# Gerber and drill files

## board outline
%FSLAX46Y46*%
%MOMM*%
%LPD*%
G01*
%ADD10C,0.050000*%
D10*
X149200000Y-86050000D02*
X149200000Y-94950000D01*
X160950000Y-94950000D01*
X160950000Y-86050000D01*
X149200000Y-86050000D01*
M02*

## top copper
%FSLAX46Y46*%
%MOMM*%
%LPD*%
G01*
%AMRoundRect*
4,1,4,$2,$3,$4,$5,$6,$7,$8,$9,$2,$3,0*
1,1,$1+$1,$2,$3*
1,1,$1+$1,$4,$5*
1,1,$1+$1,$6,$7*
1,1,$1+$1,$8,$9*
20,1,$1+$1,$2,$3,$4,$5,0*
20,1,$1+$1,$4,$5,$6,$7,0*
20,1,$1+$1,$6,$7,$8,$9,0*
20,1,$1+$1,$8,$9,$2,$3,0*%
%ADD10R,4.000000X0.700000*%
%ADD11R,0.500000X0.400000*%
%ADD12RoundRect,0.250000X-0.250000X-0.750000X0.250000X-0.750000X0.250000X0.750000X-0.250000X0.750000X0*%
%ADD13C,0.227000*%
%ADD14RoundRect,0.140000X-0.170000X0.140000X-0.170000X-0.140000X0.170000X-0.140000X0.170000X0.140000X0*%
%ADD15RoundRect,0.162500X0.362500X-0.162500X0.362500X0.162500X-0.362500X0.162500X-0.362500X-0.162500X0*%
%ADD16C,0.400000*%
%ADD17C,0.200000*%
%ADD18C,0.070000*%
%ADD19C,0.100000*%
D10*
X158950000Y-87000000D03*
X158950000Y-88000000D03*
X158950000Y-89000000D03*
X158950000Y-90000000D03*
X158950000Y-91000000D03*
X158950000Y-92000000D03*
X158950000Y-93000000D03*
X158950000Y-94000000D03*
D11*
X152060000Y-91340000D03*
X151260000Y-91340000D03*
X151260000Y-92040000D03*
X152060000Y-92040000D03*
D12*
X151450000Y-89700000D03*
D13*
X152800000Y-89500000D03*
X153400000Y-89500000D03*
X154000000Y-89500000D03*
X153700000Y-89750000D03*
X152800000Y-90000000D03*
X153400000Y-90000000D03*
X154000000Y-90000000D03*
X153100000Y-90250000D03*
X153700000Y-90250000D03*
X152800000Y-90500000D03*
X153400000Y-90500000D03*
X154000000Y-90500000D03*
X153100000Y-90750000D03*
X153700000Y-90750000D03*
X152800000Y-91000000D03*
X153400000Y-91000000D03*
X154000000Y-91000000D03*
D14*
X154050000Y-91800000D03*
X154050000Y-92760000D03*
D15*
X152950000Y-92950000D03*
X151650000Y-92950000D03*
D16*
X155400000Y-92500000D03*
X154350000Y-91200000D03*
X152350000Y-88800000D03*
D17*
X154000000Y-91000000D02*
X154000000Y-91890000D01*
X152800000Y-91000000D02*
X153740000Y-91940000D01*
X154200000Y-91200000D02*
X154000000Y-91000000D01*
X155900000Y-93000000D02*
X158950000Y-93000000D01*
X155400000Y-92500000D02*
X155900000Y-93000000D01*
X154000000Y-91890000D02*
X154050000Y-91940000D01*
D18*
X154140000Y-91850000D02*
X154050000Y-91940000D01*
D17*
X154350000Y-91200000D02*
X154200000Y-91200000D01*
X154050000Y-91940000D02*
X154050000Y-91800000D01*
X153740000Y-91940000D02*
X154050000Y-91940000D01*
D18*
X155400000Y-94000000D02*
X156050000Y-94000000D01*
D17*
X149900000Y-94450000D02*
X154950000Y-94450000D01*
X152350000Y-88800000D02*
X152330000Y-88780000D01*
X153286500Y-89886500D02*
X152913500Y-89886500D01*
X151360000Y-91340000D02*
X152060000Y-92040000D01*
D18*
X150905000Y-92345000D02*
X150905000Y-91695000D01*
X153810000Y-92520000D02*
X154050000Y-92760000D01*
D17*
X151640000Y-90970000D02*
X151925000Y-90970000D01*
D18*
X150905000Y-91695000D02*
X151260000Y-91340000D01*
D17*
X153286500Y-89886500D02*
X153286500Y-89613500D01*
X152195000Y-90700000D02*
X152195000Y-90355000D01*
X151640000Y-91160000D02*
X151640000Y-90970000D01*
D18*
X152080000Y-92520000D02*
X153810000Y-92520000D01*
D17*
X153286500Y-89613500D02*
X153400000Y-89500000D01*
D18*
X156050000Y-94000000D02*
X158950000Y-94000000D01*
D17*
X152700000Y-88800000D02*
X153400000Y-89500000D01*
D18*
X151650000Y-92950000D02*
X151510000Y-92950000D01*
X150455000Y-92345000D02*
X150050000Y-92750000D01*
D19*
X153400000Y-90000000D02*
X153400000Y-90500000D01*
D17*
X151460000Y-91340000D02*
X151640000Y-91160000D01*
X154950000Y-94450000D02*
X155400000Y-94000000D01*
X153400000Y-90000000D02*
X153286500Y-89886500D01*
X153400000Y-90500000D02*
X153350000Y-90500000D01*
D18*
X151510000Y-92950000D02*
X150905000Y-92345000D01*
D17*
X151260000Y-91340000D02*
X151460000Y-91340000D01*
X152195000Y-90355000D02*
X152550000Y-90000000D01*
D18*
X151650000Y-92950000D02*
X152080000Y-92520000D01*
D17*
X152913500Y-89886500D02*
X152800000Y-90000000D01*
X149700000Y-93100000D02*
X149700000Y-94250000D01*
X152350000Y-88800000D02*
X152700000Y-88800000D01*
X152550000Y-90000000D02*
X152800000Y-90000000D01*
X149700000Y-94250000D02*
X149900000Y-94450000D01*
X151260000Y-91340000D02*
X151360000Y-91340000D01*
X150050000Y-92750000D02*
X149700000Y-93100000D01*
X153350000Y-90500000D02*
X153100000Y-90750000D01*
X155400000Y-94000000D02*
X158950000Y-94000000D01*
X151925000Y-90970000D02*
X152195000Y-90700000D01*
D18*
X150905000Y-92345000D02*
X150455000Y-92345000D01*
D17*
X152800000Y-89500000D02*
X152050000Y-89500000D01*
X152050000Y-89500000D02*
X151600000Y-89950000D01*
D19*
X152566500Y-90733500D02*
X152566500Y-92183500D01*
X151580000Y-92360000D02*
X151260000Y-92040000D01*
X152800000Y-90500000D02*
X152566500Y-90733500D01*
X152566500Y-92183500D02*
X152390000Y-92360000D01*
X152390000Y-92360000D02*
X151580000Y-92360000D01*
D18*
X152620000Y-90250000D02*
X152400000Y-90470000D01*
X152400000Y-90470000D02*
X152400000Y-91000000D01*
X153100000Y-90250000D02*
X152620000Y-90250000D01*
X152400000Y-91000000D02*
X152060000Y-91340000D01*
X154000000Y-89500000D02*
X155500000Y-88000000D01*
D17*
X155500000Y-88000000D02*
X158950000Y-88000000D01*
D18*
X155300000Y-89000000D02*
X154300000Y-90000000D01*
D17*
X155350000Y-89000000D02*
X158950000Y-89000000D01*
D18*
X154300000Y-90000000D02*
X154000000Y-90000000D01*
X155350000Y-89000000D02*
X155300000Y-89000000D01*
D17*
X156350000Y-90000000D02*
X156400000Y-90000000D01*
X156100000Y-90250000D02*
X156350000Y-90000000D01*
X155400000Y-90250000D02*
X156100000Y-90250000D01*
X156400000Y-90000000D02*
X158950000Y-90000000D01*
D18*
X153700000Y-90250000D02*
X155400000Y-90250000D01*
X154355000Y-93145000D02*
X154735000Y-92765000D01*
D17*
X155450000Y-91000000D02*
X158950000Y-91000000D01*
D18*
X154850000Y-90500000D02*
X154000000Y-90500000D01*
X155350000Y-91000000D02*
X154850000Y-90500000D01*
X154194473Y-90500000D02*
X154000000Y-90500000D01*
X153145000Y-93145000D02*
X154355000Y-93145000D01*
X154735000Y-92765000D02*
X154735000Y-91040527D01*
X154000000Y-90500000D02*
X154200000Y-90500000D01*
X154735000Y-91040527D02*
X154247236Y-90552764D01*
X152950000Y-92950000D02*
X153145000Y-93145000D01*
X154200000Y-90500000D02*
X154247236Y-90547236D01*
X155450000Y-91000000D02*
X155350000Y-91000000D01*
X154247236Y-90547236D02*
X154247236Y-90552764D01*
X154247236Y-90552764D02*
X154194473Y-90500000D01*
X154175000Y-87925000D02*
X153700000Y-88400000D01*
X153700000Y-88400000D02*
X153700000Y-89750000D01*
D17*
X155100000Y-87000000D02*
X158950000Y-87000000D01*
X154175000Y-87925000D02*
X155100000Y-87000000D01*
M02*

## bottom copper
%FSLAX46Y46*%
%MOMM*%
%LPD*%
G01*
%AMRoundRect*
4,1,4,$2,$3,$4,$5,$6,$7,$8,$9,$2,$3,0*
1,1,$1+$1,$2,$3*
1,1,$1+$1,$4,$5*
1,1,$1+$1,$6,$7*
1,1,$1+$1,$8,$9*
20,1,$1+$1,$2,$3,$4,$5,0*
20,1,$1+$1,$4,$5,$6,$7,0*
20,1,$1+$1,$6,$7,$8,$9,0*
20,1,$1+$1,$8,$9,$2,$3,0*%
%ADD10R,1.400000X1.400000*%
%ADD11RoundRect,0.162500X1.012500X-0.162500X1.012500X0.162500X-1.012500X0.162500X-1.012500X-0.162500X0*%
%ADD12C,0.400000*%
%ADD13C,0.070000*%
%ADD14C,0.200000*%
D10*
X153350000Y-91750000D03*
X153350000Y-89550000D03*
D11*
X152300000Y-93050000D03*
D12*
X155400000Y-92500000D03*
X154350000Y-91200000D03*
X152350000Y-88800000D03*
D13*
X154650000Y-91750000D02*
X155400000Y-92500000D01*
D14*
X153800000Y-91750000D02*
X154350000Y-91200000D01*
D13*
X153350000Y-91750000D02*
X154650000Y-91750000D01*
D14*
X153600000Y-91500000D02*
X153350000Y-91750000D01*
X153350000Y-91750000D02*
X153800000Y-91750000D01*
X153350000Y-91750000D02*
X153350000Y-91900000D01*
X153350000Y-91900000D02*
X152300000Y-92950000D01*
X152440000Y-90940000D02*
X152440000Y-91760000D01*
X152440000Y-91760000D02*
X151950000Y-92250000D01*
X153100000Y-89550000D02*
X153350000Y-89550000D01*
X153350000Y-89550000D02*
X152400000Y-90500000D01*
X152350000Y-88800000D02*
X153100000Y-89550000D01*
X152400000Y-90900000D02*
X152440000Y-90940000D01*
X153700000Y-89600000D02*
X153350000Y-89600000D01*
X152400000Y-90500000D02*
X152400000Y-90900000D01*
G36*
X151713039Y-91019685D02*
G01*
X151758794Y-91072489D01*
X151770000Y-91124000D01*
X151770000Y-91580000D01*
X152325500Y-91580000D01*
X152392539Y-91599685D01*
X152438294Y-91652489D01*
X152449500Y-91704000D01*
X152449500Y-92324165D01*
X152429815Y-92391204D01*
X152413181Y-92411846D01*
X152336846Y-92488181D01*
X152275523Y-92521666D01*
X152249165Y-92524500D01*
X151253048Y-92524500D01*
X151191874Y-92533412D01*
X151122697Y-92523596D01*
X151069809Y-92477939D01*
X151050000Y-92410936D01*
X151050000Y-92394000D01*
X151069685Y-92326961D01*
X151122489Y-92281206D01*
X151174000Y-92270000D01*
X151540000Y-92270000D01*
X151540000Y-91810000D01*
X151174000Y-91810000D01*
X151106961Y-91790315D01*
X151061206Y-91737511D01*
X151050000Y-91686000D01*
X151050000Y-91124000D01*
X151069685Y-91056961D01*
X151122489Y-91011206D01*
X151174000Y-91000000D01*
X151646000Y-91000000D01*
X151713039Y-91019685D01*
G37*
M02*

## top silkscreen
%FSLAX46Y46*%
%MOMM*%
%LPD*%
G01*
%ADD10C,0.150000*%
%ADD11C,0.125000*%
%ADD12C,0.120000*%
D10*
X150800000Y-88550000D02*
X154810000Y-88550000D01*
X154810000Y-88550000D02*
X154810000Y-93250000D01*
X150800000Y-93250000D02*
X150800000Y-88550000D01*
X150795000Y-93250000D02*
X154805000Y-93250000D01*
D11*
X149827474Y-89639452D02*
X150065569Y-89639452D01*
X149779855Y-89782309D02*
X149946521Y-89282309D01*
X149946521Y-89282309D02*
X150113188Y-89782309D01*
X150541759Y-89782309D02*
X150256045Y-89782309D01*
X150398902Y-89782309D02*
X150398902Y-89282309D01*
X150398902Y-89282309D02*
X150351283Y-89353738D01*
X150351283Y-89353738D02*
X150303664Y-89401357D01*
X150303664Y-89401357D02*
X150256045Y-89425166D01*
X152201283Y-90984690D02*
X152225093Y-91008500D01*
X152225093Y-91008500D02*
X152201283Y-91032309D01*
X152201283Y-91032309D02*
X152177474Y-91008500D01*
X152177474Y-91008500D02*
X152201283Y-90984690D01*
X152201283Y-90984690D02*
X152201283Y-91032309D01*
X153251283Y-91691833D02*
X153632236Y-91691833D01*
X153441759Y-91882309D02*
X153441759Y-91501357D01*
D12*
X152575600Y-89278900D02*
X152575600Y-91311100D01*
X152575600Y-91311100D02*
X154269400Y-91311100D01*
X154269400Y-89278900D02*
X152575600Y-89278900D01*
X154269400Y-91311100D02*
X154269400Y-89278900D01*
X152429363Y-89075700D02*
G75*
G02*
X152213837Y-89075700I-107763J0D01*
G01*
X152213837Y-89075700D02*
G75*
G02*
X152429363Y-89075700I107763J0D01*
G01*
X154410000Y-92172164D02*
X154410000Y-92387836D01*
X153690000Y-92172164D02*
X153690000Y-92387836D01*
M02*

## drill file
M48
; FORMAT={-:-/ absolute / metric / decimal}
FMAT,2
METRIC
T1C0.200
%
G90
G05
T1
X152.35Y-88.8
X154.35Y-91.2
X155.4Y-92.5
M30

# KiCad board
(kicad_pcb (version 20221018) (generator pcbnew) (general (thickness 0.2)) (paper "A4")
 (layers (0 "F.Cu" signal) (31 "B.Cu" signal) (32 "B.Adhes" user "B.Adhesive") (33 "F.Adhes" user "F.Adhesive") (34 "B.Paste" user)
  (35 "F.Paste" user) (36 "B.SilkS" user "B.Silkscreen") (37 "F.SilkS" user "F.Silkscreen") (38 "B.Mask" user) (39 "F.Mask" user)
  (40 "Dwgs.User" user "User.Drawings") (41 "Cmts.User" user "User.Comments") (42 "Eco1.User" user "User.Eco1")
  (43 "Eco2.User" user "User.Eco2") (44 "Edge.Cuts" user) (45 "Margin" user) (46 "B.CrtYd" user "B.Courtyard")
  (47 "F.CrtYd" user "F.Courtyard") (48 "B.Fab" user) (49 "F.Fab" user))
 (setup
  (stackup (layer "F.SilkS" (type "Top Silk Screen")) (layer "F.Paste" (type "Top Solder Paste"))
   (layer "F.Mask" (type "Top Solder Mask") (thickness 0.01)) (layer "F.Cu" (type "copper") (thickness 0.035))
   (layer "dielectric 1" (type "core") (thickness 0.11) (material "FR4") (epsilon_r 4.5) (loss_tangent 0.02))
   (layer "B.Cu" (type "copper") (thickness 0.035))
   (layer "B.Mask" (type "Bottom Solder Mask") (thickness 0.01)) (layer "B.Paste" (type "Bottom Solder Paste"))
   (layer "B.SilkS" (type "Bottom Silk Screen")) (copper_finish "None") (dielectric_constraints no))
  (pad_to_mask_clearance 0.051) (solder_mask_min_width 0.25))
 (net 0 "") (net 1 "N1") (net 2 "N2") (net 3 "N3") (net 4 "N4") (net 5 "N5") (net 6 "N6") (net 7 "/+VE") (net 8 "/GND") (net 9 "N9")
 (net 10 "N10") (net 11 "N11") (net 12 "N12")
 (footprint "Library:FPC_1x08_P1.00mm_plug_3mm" (layer "F.Cu") (at 156.95 90.5)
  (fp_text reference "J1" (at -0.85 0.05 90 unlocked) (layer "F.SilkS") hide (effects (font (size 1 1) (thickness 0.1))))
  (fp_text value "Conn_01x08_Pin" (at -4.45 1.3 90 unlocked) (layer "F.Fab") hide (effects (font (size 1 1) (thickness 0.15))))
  (pad "1" connect rect (at 2 -3.5) (size 4 0.7) (layers "F.Cu" "F.Mask") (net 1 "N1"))
  (pad "2" connect rect (at 2 -2.5) (size 4 0.7) (layers "F.Cu" "F.Mask") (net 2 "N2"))
  (pad "3" connect rect (at 2 -1.5) (size 4 0.7) (layers "F.Cu" "F.Mask") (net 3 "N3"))
  (pad "4" connect rect (at 2 -0.5) (size 4 0.7) (layers "F.Cu" "F.Mask") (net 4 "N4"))
  (pad "5" connect rect (at 2 0.5) (size 4 0.7) (layers "F.Cu" "F.Mask") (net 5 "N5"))
  (pad "6" connect rect (at 2 1.5) (size 4 0.7) (layers "F.Cu" "F.Mask") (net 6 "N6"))
  (pad "7" connect rect (at 2 2.5) (size 4 0.7) (layers "F.Cu" "F.Mask") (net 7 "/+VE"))
  (pad "8" connect rect (at 2 3.5) (size 4 0.7) (layers "F.Cu" "F.Mask") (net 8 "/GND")))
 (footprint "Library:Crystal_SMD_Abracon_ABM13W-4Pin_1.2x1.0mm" (layer "F.Cu") (at 151.66 91.69 180)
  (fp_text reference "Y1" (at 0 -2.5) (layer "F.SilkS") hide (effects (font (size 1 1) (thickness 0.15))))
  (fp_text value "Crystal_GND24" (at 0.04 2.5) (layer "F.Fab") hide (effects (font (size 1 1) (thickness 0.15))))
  (pad "1" smd rect (at -0.4 0.35 180) (size 0.5 0.4) (layers "F.Cu" "F.Paste" "F.Mask") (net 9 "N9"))
  (pad "2" smd rect (at 0.4 0.35 180) (size 0.5 0.4) (layers "F.Cu" "F.Paste" "F.Mask") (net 8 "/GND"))
  (pad "3" smd rect (at 0.4 -0.35 180) (size 0.5 0.4) (layers "F.Cu" "F.Paste" "F.Mask") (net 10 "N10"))
  (pad "4" smd rect (at -0.4 -0.35 180) (size 0.5 0.4) (layers "F.Cu" "F.Paste" "F.Mask") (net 8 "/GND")))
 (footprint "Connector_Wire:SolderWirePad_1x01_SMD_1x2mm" (layer "F.Cu") (at 151.45 89.7)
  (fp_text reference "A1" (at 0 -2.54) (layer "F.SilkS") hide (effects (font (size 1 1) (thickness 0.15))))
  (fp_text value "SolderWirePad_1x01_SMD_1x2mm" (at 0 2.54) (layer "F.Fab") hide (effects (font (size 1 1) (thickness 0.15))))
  (pad "1" smd roundrect (at 0 0) (size 1 2) (layers "F.Cu" "F.Paste" "F.Mask") (roundrect_rratio 0.25) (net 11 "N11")))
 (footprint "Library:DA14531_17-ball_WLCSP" (layer "F.Cu") (at 153.422 90.295)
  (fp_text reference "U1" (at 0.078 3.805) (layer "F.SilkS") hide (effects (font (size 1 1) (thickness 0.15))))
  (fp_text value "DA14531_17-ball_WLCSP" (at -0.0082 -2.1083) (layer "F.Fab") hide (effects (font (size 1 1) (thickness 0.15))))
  (fp_line (start -0.8464 -1.0161) (end -0.8464 1.0161) (stroke (width 0.12) (type solid)) (layer "F.SilkS"))
  (fp_line (start -0.8464 1.0161) (end 0.8474 1.0161) (stroke (width 0.12) (type solid)) (layer "F.SilkS"))
  (fp_line (start 0.8474 -1.0161) (end -0.8464 -1.0161) (stroke (width 0.12) (type solid)) (layer "F.SilkS"))
  (fp_line (start 0.8474 1.0161) (end 0.8474 -1.0161) (stroke (width 0.12) (type solid)) (layer "F.SilkS"))
  (fp_circle (center -1.1004 -1.2193) (end -1.0242 -1.1431) (stroke (width 0.12) (type solid)) (fill none) (layer "F.SilkS"))
  (pad "A1" smd circle (at -0.622 -0.795) (size 0.227 0.227) (layers "F.Cu" "F.Paste" "F.Mask") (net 11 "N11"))
  (pad "A3" smd circle (at -0.022 -0.795) (size 0.227 0.227) (layers "F.Cu" "F.Paste" "F.Mask") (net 8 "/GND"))
  (pad "A5" smd circle (at 0.578 -0.795) (size 0.227 0.227) (layers "F.Cu" "F.Paste" "F.Mask") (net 2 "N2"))
  (pad "B4" smd circle (at 0.278 -0.545) (size 0.227 0.227) (layers "F.Cu" "F.Paste" "F.Mask") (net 1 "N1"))
  (pad "C1" smd circle (at -0.622 -0.295) (size 0.227 0.227) (layers "F.Cu" "F.Paste" "F.Mask") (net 8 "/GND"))
  (pad "C3" smd circle (at -0.022 -0.295) (size 0.227 0.227) (layers "F.Cu" "F.Paste" "F.Mask") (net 8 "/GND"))
  (pad "C5" smd circle (at 0.578 -0.295) (size 0.227 0.227) (layers "F.Cu" "F.Paste" "F.Mask") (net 3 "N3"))
  (pad "D2" smd circle (at -0.322 -0.045) (size 0.227 0.227) (layers "F.Cu" "F.Paste" "F.Mask") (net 9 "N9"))
  (pad "D4" smd circle (at 0.278 -0.045) (size 0.227 0.227) (layers "F.Cu" "F.Paste" "F.Mask") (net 4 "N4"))
  (pad "E1" smd circle (at -0.622 0.205) (size 0.227 0.227) (layers "F.Cu" "F.Paste" "F.Mask") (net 10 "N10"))
  (pad "E3" smd circle (at -0.022 0.205) (size 0.227 0.227) (layers "F.Cu" "F.Paste" "F.Mask") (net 8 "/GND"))
  (pad "E5" smd circle (at 0.578 0.205) (size 0.227 0.227) (layers "F.Cu" "F.Paste" "F.Mask") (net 5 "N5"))
  (pad "F2" smd circle (at -0.322 0.455) (size 0.227 0.227) (layers "F.Cu" "F.Paste" "F.Mask") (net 8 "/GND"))
  (pad "F4" smd circle (at 0.278 0.455) (size 0.227 0.227) (layers "F.Cu" "F.Paste" "F.Mask") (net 6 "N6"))
  (pad "G1" smd circle (at -0.622 0.705) (size 0.227 0.227) (layers "F.Cu" "F.Paste" "F.Mask") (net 7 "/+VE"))
  (pad "G3" smd circle (at -0.022 0.705) (size 0.227 0.227) (layers "F.Cu" "F.Paste" "F.Mask") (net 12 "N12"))
  (pad "G5" smd circle (at 0.578 0.705) (size 0.227 0.227) (layers "F.Cu" "F.Paste" "F.Mask") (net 7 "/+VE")))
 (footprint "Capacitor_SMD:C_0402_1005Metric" (layer "F.Cu") (at 154.05 92.28 -90)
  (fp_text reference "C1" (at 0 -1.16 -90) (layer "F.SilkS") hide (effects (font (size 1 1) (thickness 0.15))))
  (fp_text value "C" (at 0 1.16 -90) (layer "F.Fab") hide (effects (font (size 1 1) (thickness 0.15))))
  (fp_line (start -0.107836 -0.36) (end 0.107836 -0.36) (stroke (width 0.12) (type solid)) (layer "F.SilkS"))
  (fp_line (start -0.107836 0.36) (end 0.107836 0.36) (stroke (width 0.12) (type solid)) (layer "F.SilkS"))
  (pad "1" smd roundrect (at -0.48 0 270) (size 0.56 0.62) (layers "F.Cu" "F.Paste" "F.Mask") (roundrect_rratio 0.25) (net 7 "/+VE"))
  (pad "2" smd roundrect (at 0.48 0 270) (size 0.56 0.62) (layers "F.Cu" "F.Paste" "F.Mask") (roundrect_rratio 0.25) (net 8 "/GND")))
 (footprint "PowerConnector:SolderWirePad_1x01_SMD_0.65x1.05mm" (layer "F.Cu") (at 152.95 92.95 90)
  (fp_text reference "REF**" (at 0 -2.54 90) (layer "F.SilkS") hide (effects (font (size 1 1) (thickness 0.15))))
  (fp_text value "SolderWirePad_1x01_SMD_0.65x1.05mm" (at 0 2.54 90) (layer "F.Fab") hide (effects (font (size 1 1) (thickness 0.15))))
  (pad "1" smd roundrect (at 0 0 90) (size 0.65 1.05) (layers "F.Cu" "F.Paste" "F.Mask") (roundrect_rratio 0.25) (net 5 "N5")))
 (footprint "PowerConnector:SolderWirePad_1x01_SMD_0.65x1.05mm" (layer "F.Cu") (at 151.65 92.95 90)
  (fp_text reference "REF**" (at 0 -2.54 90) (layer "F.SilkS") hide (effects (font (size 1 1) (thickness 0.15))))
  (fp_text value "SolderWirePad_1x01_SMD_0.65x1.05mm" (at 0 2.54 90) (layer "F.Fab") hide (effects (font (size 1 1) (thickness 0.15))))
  (pad "1" smd roundrect (at 0 0 90) (size 0.65 1.05) (layers "F.Cu" "F.Paste" "F.Mask") (roundrect_rratio 0.25) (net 8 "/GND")))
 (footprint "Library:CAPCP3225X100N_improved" (layer "B.Cu") (at 153.35 90.65 90)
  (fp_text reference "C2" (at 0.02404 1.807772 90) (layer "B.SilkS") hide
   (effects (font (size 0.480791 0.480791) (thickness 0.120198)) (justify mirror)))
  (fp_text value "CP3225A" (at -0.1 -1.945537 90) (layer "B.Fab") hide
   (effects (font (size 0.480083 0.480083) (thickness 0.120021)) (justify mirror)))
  (pad "1" smd rect (at -1.1 0 270) (size 1.4 1.4) (layers "B.Cu" "B.Paste" "B.Mask") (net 7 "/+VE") (solder_mask_margin 0.102))
  (pad "2" smd rect (at 1.1 0 270) (size 1.4 1.4) (layers "B.Cu" "B.Paste" "B.Mask") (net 8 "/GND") (solder_mask_margin 0.102)))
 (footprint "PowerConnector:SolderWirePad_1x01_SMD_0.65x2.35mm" (layer "B.Cu") (at 152.3 93.05 90)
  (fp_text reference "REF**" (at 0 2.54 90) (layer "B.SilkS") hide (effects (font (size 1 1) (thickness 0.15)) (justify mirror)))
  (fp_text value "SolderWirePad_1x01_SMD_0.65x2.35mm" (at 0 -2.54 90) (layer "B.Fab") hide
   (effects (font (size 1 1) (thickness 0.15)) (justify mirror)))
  (pad "1" smd roundrect (at 0 0 90) (size 0.65 2.35) (layers "B.Cu" "B.Paste" "B.Mask") (roundrect_rratio 0.25) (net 7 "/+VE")))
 (gr_line (start 150.8 88.55) (end 154.81 88.55) (stroke (width 0.15) (type default)) (layer "F.SilkS"))
 (gr_line (start 154.81 88.55) (end 154.81 93.25) (stroke (width 0.15) (type default)) (layer "F.SilkS"))
 (gr_line (start 150.8 93.25) (end 150.8 88.55) (stroke (width 0.15) (type default)) (layer "F.SilkS"))
 (gr_line (start 150.795 93.25) (end 154.805 93.25) (stroke (width 0.15) (type default)) (layer "F.SilkS"))
 (gr_poly
  (pts (xy 149.2 86.05) (xy 149.2 94.95) (xy 160.95 94.95) (xy 160.95 86.05)) (stroke (width 0.05) (type solid)) (fill none)
  (layer "Edge.Cuts"))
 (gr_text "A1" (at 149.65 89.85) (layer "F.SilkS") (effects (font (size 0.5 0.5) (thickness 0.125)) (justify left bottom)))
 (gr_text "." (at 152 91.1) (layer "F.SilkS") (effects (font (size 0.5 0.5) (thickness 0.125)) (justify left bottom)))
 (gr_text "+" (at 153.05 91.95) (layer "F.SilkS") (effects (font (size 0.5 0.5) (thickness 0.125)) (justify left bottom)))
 (segment (start 154 91) (end 154 91.89) (width 0.2) (layer "F.Cu") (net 7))
 (segment (start 152.8 91) (end 153.74 91.94) (width 0.2) (layer "F.Cu") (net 7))
 (segment (start 154.2 91.2) (end 154 91) (width 0.2) (layer "F.Cu") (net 7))
 (segment (start 155.9 93) (end 158.95 93) (width 0.2) (layer "F.Cu") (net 7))
 (segment (start 155.4 92.5) (end 155.9 93) (width 0.2) (layer "F.Cu") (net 7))
 (segment (start 154 91.89) (end 154.05 91.94) (width 0.2) (layer "F.Cu") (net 7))
 (segment (start 154.14 91.85) (end 154.05 91.94) (width 0.07) (layer "F.Cu") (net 7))
 (segment (start 154.35 91.2) (end 154.2 91.2) (width 0.2) (layer "F.Cu") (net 7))
 (segment (start 154.05 91.94) (end 154.05 91.8) (width 0.2) (layer "F.Cu") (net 7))
 (segment (start 153.74 91.94) (end 154.05 91.94) (width 0.2) (layer "F.Cu") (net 7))
 (via (at 155.4 92.5) (size 0.4) (drill 0.2) (layers "F.Cu" "B.Cu") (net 7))
 (via (at 154.35 91.2) (size 0.4) (drill 0.2) (layers "F.Cu" "B.Cu") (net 7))
 (segment (start 154.65 91.75) (end 155.4 92.5) (width 0.07) (layer "B.Cu") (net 7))
 (segment (start 153.8 91.75) (end 154.35 91.2) (width 0.2) (layer "B.Cu") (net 7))
 (segment (start 153.35 91.75) (end 154.65 91.75) (width 0.07) (layer "B.Cu") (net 7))
 (segment (start 153.6 91.5) (end 153.35 91.75) (width 0.2) (layer "B.Cu") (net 7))
 (segment (start 153.35 91.75) (end 153.8 91.75) (width 0.2) (layer "B.Cu") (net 7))
 (segment (start 153.35 91.75) (end 153.35 91.9) (width 0.2) (layer "B.Cu") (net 7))
 (segment (start 153.35 91.9) (end 152.3 92.95) (width 0.2) (layer "B.Cu") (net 7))
 (segment (start 155.4 94) (end 156.05 94) (width 0.07) (layer "F.Cu") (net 8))
 (segment (start 149.9 94.45) (end 154.95 94.45) (width 0.2) (layer "F.Cu") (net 8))
 (segment (start 152.35 88.8) (end 152.33 88.78) (width 0.2) (layer "F.Cu") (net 8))
 (segment (start 153.2865 89.8865) (end 152.9135 89.8865) (width 0.2) (layer "F.Cu") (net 8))
 (segment (start 151.36 91.34) (end 152.06 92.04) (width 0.2) (layer "F.Cu") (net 8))
 (segment (start 150.905 92.345) (end 150.905 91.695) (width 0.07) (layer "F.Cu") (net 8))
 (segment (start 153.81 92.52) (end 154.05 92.76) (width 0.07) (layer "F.Cu") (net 8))
 (segment (start 151.64 90.97) (end 151.925 90.97) (width 0.2) (layer "F.Cu") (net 8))
 (segment (start 150.905 91.695) (end 151.26 91.34) (width 0.07) (layer "F.Cu") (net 8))
 (segment (start 153.2865 89.8865) (end 153.2865 89.6135) (width 0.2) (layer "F.Cu") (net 8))
 (segment (start 152.195 90.7) (end 152.195 90.355) (width 0.2) (layer "F.Cu") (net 8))
 (segment (start 151.64 91.16) (end 151.64 90.97) (width 0.2) (layer "F.Cu") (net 8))
 (segment (start 152.08 92.52) (end 153.81 92.52) (width 0.07) (layer "F.Cu") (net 8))
 (segment (start 153.2865 89.6135) (end 153.4 89.5) (width 0.2) (layer "F.Cu") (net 8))
 (segment (start 156.05 94) (end 158.95 94) (width 0.07) (layer "F.Cu") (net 8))
 (segment (start 152.7 88.8) (end 153.4 89.5) (width 0.2) (layer "F.Cu") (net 8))
 (segment (start 151.65 92.95) (end 151.51 92.95) (width 0.07) (layer "F.Cu") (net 8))
 (segment (start 150.455 92.345) (end 150.05 92.75) (width 0.07) (layer "F.Cu") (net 8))
 (segment (start 153.4 90) (end 153.4 90.5) (width 0.1) (layer "F.Cu") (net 8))
 (segment (start 151.46 91.34) (end 151.64 91.16) (width 0.2) (layer "F.Cu") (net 8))
 (segment (start 154.95 94.45) (end 155.4 94) (width 0.2) (layer "F.Cu") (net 8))
 (segment (start 153.4 90) (end 153.2865 89.8865) (width 0.2) (layer "F.Cu") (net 8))
 (segment (start 153.4 90.5) (end 153.35 90.5) (width 0.2) (layer "F.Cu") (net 8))
 (segment (start 151.51 92.95) (end 150.905 92.345) (width 0.07) (layer "F.Cu") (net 8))
 (segment (start 151.26 91.34) (end 151.46 91.34) (width 0.2) (layer "F.Cu") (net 8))
 (segment (start 152.195 90.355) (end 152.55 90) (width 0.2) (layer "F.Cu") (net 8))
 (segment (start 151.65 92.95) (end 152.08 92.52) (width 0.07) (layer "F.Cu") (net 8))
 (segment (start 152.9135 89.8865) (end 152.8 90) (width 0.2) (layer "F.Cu") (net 8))
 (segment (start 149.7 93.1) (end 149.7 94.25) (width 0.2) (layer "F.Cu") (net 8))
 (segment (start 152.35 88.8) (end 152.7 88.8) (width 0.2) (layer "F.Cu") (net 8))
 (segment (start 152.55 90) (end 152.8 90) (width 0.2) (layer "F.Cu") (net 8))
 (segment (start 149.7 94.25) (end 149.9 94.45) (width 0.2) (layer "F.Cu") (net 8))
 (segment (start 151.26 91.34) (end 151.36 91.34) (width 0.2) (layer "F.Cu") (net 8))
 (segment (start 150.05 92.75) (end 149.7 93.1) (width 0.2) (layer "F.Cu") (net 8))
 (segment (start 153.35 90.5) (end 153.1 90.75) (width 0.2) (layer "F.Cu") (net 8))
 (segment (start 155.4 94) (end 158.95 94) (width 0.2) (layer "F.Cu") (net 8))
 (segment (start 151.925 90.97) (end 152.195 90.7) (width 0.2) (layer "F.Cu") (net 8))
 (segment (start 150.905 92.345) (end 150.455 92.345) (width 0.07) (layer "F.Cu") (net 8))
 (via (at 152.35 88.8) (size 0.4) (drill 0.2) (layers "F.Cu" "B.Cu") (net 8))
 (segment (start 152.44 90.94) (end 152.44 91.76) (width 0.2) (layer "B.Cu") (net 8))
 (segment (start 152.44 91.76) (end 151.95 92.25) (width 0.2) (layer "B.Cu") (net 8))
 (segment (start 153.1 89.55) (end 153.35 89.55) (width 0.2) (layer "B.Cu") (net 8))
 (segment (start 153.35 89.55) (end 152.4 90.5) (width 0.2) (layer "B.Cu") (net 8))
 (segment (start 152.35 88.8) (end 153.1 89.55) (width 0.2) (layer "B.Cu") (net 8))
 (segment (start 152.4 90.9) (end 152.44 90.94) (width 0.2) (layer "B.Cu") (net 8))
 (segment (start 153.7 89.6) (end 153.35 89.6) (width 0.2) (layer "B.Cu") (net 8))
 (segment (start 152.4 90.5) (end 152.4 90.9) (width 0.2) (layer "B.Cu") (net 8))
 (segment (start 152.8 89.5) (end 152.05 89.5) (width 0.2) (layer "F.Cu") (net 11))
 (segment (start 152.05 89.5) (end 151.6 89.95) (width 0.2) (layer "F.Cu") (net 11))
 (segment (start 152.5665 90.7335) (end 152.5665 92.1835) (width 0.1) (layer "F.Cu") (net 10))
 (segment (start 151.58 92.36) (end 151.26 92.04) (width 0.1) (layer "F.Cu") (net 10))
 (segment (start 152.8 90.5) (end 152.5665 90.7335) (width 0.1) (layer "F.Cu") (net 10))
 (segment (start 152.5665 92.1835) (end 152.39 92.36) (width 0.1) (layer "F.Cu") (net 10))
 (segment (start 152.39 92.36) (end 151.58 92.36) (width 0.1) (layer "F.Cu") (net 10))
 (segment (start 152.62 90.25) (end 152.4 90.47) (width 0.07) (layer "F.Cu") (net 9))
 (segment (start 152.4 90.47) (end 152.4 91) (width 0.07) (layer "F.Cu") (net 9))
 (segment (start 153.1 90.25) (end 152.62 90.25) (width 0.07) (layer "F.Cu") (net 9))
 (segment (start 152.4 91) (end 152.06 91.34) (width 0.07) (layer "F.Cu") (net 9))
 (segment (start 154 89.5) (end 155.5 88) (width 0.07) (layer "F.Cu") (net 2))
 (segment (start 155.5 88) (end 158.95 88) (width 0.2) (layer "F.Cu") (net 2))
 (segment (start 155.3 89) (end 154.3 90) (width 0.07) (layer "F.Cu") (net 3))
 (segment (start 155.35 89) (end 158.95 89) (width 0.2) (layer "F.Cu") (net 3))
 (segment (start 154.3 90) (end 154 90) (width 0.07) (layer "F.Cu") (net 3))
 (segment (start 155.35 89) (end 155.3 89) (width 0.07) (layer "F.Cu") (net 3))
 (segment (start 156.35 90) (end 156.4 90) (width 0.2) (layer "F.Cu") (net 4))
 (segment (start 156.1 90.25) (end 156.35 90) (width 0.2) (layer "F.Cu") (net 4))
 (segment (start 155.4 90.25) (end 156.1 90.25) (width 0.2) (layer "F.Cu") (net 4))
 (segment (start 156.4 90) (end 158.95 90) (width 0.2) (layer "F.Cu") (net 4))
 (segment (start 153.7 90.25) (end 155.4 90.25) (width 0.07) (layer "F.Cu") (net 4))
 (segment (start 154.355 93.145) (end 154.735 92.765) (width 0.07) (layer "F.Cu") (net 5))
 (segment (start 155.45 91) (end 158.95 91) (width 0.2) (layer "F.Cu") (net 5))
 (segment (start 154.85 90.5) (end 154 90.5) (width 0.07) (layer "F.Cu") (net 5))
 (segment (start 155.35 91) (end 154.85 90.5) (width 0.07) (layer "F.Cu") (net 5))
 (segment (start 154.194473 90.5) (end 154 90.5) (width 0.07) (layer "F.Cu") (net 5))
 (segment (start 153.145 93.145) (end 154.355 93.145) (width 0.07) (layer "F.Cu") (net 5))
 (segment (start 154.735 92.765) (end 154.735 91.040527) (width 0.07) (layer "F.Cu") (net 5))
 (segment (start 154 90.5) (end 154.2 90.5) (width 0.07) (layer "F.Cu") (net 5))
 (segment (start 154.735 91.040527) (end 154.247236 90.552764) (width 0.07) (layer "F.Cu") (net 5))
 (segment (start 152.95 92.95) (end 153.145 93.145) (width 0.07) (layer "F.Cu") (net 5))
 (segment (start 154.2 90.5) (end 154.247236 90.547236) (width 0.07) (layer "F.Cu") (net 5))
 (segment (start 155.45 91) (end 155.35 91) (width 0.07) (layer "F.Cu") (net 5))
 (segment (start 154.247236 90.547236) (end 154.247236 90.552764) (width 0.07) (layer "F.Cu") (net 5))
 (segment (start 154.247236 90.552764) (end 154.194473 90.5) (width 0.07) (layer "F.Cu") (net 5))
 (segment (start 154.175 87.925) (end 153.7 88.4) (width 0.07) (layer "F.Cu") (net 1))
 (segment (start 153.7 88.4) (end 153.7 89.75) (width 0.07) (layer "F.Cu") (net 1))
 (segment (start 155.1 87) (end 158.95 87) (width 0.2) (layer "F.Cu") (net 1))
 (segment (start 154.175 87.925) (end 155.1 87) (width 0.2) (layer "F.Cu") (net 1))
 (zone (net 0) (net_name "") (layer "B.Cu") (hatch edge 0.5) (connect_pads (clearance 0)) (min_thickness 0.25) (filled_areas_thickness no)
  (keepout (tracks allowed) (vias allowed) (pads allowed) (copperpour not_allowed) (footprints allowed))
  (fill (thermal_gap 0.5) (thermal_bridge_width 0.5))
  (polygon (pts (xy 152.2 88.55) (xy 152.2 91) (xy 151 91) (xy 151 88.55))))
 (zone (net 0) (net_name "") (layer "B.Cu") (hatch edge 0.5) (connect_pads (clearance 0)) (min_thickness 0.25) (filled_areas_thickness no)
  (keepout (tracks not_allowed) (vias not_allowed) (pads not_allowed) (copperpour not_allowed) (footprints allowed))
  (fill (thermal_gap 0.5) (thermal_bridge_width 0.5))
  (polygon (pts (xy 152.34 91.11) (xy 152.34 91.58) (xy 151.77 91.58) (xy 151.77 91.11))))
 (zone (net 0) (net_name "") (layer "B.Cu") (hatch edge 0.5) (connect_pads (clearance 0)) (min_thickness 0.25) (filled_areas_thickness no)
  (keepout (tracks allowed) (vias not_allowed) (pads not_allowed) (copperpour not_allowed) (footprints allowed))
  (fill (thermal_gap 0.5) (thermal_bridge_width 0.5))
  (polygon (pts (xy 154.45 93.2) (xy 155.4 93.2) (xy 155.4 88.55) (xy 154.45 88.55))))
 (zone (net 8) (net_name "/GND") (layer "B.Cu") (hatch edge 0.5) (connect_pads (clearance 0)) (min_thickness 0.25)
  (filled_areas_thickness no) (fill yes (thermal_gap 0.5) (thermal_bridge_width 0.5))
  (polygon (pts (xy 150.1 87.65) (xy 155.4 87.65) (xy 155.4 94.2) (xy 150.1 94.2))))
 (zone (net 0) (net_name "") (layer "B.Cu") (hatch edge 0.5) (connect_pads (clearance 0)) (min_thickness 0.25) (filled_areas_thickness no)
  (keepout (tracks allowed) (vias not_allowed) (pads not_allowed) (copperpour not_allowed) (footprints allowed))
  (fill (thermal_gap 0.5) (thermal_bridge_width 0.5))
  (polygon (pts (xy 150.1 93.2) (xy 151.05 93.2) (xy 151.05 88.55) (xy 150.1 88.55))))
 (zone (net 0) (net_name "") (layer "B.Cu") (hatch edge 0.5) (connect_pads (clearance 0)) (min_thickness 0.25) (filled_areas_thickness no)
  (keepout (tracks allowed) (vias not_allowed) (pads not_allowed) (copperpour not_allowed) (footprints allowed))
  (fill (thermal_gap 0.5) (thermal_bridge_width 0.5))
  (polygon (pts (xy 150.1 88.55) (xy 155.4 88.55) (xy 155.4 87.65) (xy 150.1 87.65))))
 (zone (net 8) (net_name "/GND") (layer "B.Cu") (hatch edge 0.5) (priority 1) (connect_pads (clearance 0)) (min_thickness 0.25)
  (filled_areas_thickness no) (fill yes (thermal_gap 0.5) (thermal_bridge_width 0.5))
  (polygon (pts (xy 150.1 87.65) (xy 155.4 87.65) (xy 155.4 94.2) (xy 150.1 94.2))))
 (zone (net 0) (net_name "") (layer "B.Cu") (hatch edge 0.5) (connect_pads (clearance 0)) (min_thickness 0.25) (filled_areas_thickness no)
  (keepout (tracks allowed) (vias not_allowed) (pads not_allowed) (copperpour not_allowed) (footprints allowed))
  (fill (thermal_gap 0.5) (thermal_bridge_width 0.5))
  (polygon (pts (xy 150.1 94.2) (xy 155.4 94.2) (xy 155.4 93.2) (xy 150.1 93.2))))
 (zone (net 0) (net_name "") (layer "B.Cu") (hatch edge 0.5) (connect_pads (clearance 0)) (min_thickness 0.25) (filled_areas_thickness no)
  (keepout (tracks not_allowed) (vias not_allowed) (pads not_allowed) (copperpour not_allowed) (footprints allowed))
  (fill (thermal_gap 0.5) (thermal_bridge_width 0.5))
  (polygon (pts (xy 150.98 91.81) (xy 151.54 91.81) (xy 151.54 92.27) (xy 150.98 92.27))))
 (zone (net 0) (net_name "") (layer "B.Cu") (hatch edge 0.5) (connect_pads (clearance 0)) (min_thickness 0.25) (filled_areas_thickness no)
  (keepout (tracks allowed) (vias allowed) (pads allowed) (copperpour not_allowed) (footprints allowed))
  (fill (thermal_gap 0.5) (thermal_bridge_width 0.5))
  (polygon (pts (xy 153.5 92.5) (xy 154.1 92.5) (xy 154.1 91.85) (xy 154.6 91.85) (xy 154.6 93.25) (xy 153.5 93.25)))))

